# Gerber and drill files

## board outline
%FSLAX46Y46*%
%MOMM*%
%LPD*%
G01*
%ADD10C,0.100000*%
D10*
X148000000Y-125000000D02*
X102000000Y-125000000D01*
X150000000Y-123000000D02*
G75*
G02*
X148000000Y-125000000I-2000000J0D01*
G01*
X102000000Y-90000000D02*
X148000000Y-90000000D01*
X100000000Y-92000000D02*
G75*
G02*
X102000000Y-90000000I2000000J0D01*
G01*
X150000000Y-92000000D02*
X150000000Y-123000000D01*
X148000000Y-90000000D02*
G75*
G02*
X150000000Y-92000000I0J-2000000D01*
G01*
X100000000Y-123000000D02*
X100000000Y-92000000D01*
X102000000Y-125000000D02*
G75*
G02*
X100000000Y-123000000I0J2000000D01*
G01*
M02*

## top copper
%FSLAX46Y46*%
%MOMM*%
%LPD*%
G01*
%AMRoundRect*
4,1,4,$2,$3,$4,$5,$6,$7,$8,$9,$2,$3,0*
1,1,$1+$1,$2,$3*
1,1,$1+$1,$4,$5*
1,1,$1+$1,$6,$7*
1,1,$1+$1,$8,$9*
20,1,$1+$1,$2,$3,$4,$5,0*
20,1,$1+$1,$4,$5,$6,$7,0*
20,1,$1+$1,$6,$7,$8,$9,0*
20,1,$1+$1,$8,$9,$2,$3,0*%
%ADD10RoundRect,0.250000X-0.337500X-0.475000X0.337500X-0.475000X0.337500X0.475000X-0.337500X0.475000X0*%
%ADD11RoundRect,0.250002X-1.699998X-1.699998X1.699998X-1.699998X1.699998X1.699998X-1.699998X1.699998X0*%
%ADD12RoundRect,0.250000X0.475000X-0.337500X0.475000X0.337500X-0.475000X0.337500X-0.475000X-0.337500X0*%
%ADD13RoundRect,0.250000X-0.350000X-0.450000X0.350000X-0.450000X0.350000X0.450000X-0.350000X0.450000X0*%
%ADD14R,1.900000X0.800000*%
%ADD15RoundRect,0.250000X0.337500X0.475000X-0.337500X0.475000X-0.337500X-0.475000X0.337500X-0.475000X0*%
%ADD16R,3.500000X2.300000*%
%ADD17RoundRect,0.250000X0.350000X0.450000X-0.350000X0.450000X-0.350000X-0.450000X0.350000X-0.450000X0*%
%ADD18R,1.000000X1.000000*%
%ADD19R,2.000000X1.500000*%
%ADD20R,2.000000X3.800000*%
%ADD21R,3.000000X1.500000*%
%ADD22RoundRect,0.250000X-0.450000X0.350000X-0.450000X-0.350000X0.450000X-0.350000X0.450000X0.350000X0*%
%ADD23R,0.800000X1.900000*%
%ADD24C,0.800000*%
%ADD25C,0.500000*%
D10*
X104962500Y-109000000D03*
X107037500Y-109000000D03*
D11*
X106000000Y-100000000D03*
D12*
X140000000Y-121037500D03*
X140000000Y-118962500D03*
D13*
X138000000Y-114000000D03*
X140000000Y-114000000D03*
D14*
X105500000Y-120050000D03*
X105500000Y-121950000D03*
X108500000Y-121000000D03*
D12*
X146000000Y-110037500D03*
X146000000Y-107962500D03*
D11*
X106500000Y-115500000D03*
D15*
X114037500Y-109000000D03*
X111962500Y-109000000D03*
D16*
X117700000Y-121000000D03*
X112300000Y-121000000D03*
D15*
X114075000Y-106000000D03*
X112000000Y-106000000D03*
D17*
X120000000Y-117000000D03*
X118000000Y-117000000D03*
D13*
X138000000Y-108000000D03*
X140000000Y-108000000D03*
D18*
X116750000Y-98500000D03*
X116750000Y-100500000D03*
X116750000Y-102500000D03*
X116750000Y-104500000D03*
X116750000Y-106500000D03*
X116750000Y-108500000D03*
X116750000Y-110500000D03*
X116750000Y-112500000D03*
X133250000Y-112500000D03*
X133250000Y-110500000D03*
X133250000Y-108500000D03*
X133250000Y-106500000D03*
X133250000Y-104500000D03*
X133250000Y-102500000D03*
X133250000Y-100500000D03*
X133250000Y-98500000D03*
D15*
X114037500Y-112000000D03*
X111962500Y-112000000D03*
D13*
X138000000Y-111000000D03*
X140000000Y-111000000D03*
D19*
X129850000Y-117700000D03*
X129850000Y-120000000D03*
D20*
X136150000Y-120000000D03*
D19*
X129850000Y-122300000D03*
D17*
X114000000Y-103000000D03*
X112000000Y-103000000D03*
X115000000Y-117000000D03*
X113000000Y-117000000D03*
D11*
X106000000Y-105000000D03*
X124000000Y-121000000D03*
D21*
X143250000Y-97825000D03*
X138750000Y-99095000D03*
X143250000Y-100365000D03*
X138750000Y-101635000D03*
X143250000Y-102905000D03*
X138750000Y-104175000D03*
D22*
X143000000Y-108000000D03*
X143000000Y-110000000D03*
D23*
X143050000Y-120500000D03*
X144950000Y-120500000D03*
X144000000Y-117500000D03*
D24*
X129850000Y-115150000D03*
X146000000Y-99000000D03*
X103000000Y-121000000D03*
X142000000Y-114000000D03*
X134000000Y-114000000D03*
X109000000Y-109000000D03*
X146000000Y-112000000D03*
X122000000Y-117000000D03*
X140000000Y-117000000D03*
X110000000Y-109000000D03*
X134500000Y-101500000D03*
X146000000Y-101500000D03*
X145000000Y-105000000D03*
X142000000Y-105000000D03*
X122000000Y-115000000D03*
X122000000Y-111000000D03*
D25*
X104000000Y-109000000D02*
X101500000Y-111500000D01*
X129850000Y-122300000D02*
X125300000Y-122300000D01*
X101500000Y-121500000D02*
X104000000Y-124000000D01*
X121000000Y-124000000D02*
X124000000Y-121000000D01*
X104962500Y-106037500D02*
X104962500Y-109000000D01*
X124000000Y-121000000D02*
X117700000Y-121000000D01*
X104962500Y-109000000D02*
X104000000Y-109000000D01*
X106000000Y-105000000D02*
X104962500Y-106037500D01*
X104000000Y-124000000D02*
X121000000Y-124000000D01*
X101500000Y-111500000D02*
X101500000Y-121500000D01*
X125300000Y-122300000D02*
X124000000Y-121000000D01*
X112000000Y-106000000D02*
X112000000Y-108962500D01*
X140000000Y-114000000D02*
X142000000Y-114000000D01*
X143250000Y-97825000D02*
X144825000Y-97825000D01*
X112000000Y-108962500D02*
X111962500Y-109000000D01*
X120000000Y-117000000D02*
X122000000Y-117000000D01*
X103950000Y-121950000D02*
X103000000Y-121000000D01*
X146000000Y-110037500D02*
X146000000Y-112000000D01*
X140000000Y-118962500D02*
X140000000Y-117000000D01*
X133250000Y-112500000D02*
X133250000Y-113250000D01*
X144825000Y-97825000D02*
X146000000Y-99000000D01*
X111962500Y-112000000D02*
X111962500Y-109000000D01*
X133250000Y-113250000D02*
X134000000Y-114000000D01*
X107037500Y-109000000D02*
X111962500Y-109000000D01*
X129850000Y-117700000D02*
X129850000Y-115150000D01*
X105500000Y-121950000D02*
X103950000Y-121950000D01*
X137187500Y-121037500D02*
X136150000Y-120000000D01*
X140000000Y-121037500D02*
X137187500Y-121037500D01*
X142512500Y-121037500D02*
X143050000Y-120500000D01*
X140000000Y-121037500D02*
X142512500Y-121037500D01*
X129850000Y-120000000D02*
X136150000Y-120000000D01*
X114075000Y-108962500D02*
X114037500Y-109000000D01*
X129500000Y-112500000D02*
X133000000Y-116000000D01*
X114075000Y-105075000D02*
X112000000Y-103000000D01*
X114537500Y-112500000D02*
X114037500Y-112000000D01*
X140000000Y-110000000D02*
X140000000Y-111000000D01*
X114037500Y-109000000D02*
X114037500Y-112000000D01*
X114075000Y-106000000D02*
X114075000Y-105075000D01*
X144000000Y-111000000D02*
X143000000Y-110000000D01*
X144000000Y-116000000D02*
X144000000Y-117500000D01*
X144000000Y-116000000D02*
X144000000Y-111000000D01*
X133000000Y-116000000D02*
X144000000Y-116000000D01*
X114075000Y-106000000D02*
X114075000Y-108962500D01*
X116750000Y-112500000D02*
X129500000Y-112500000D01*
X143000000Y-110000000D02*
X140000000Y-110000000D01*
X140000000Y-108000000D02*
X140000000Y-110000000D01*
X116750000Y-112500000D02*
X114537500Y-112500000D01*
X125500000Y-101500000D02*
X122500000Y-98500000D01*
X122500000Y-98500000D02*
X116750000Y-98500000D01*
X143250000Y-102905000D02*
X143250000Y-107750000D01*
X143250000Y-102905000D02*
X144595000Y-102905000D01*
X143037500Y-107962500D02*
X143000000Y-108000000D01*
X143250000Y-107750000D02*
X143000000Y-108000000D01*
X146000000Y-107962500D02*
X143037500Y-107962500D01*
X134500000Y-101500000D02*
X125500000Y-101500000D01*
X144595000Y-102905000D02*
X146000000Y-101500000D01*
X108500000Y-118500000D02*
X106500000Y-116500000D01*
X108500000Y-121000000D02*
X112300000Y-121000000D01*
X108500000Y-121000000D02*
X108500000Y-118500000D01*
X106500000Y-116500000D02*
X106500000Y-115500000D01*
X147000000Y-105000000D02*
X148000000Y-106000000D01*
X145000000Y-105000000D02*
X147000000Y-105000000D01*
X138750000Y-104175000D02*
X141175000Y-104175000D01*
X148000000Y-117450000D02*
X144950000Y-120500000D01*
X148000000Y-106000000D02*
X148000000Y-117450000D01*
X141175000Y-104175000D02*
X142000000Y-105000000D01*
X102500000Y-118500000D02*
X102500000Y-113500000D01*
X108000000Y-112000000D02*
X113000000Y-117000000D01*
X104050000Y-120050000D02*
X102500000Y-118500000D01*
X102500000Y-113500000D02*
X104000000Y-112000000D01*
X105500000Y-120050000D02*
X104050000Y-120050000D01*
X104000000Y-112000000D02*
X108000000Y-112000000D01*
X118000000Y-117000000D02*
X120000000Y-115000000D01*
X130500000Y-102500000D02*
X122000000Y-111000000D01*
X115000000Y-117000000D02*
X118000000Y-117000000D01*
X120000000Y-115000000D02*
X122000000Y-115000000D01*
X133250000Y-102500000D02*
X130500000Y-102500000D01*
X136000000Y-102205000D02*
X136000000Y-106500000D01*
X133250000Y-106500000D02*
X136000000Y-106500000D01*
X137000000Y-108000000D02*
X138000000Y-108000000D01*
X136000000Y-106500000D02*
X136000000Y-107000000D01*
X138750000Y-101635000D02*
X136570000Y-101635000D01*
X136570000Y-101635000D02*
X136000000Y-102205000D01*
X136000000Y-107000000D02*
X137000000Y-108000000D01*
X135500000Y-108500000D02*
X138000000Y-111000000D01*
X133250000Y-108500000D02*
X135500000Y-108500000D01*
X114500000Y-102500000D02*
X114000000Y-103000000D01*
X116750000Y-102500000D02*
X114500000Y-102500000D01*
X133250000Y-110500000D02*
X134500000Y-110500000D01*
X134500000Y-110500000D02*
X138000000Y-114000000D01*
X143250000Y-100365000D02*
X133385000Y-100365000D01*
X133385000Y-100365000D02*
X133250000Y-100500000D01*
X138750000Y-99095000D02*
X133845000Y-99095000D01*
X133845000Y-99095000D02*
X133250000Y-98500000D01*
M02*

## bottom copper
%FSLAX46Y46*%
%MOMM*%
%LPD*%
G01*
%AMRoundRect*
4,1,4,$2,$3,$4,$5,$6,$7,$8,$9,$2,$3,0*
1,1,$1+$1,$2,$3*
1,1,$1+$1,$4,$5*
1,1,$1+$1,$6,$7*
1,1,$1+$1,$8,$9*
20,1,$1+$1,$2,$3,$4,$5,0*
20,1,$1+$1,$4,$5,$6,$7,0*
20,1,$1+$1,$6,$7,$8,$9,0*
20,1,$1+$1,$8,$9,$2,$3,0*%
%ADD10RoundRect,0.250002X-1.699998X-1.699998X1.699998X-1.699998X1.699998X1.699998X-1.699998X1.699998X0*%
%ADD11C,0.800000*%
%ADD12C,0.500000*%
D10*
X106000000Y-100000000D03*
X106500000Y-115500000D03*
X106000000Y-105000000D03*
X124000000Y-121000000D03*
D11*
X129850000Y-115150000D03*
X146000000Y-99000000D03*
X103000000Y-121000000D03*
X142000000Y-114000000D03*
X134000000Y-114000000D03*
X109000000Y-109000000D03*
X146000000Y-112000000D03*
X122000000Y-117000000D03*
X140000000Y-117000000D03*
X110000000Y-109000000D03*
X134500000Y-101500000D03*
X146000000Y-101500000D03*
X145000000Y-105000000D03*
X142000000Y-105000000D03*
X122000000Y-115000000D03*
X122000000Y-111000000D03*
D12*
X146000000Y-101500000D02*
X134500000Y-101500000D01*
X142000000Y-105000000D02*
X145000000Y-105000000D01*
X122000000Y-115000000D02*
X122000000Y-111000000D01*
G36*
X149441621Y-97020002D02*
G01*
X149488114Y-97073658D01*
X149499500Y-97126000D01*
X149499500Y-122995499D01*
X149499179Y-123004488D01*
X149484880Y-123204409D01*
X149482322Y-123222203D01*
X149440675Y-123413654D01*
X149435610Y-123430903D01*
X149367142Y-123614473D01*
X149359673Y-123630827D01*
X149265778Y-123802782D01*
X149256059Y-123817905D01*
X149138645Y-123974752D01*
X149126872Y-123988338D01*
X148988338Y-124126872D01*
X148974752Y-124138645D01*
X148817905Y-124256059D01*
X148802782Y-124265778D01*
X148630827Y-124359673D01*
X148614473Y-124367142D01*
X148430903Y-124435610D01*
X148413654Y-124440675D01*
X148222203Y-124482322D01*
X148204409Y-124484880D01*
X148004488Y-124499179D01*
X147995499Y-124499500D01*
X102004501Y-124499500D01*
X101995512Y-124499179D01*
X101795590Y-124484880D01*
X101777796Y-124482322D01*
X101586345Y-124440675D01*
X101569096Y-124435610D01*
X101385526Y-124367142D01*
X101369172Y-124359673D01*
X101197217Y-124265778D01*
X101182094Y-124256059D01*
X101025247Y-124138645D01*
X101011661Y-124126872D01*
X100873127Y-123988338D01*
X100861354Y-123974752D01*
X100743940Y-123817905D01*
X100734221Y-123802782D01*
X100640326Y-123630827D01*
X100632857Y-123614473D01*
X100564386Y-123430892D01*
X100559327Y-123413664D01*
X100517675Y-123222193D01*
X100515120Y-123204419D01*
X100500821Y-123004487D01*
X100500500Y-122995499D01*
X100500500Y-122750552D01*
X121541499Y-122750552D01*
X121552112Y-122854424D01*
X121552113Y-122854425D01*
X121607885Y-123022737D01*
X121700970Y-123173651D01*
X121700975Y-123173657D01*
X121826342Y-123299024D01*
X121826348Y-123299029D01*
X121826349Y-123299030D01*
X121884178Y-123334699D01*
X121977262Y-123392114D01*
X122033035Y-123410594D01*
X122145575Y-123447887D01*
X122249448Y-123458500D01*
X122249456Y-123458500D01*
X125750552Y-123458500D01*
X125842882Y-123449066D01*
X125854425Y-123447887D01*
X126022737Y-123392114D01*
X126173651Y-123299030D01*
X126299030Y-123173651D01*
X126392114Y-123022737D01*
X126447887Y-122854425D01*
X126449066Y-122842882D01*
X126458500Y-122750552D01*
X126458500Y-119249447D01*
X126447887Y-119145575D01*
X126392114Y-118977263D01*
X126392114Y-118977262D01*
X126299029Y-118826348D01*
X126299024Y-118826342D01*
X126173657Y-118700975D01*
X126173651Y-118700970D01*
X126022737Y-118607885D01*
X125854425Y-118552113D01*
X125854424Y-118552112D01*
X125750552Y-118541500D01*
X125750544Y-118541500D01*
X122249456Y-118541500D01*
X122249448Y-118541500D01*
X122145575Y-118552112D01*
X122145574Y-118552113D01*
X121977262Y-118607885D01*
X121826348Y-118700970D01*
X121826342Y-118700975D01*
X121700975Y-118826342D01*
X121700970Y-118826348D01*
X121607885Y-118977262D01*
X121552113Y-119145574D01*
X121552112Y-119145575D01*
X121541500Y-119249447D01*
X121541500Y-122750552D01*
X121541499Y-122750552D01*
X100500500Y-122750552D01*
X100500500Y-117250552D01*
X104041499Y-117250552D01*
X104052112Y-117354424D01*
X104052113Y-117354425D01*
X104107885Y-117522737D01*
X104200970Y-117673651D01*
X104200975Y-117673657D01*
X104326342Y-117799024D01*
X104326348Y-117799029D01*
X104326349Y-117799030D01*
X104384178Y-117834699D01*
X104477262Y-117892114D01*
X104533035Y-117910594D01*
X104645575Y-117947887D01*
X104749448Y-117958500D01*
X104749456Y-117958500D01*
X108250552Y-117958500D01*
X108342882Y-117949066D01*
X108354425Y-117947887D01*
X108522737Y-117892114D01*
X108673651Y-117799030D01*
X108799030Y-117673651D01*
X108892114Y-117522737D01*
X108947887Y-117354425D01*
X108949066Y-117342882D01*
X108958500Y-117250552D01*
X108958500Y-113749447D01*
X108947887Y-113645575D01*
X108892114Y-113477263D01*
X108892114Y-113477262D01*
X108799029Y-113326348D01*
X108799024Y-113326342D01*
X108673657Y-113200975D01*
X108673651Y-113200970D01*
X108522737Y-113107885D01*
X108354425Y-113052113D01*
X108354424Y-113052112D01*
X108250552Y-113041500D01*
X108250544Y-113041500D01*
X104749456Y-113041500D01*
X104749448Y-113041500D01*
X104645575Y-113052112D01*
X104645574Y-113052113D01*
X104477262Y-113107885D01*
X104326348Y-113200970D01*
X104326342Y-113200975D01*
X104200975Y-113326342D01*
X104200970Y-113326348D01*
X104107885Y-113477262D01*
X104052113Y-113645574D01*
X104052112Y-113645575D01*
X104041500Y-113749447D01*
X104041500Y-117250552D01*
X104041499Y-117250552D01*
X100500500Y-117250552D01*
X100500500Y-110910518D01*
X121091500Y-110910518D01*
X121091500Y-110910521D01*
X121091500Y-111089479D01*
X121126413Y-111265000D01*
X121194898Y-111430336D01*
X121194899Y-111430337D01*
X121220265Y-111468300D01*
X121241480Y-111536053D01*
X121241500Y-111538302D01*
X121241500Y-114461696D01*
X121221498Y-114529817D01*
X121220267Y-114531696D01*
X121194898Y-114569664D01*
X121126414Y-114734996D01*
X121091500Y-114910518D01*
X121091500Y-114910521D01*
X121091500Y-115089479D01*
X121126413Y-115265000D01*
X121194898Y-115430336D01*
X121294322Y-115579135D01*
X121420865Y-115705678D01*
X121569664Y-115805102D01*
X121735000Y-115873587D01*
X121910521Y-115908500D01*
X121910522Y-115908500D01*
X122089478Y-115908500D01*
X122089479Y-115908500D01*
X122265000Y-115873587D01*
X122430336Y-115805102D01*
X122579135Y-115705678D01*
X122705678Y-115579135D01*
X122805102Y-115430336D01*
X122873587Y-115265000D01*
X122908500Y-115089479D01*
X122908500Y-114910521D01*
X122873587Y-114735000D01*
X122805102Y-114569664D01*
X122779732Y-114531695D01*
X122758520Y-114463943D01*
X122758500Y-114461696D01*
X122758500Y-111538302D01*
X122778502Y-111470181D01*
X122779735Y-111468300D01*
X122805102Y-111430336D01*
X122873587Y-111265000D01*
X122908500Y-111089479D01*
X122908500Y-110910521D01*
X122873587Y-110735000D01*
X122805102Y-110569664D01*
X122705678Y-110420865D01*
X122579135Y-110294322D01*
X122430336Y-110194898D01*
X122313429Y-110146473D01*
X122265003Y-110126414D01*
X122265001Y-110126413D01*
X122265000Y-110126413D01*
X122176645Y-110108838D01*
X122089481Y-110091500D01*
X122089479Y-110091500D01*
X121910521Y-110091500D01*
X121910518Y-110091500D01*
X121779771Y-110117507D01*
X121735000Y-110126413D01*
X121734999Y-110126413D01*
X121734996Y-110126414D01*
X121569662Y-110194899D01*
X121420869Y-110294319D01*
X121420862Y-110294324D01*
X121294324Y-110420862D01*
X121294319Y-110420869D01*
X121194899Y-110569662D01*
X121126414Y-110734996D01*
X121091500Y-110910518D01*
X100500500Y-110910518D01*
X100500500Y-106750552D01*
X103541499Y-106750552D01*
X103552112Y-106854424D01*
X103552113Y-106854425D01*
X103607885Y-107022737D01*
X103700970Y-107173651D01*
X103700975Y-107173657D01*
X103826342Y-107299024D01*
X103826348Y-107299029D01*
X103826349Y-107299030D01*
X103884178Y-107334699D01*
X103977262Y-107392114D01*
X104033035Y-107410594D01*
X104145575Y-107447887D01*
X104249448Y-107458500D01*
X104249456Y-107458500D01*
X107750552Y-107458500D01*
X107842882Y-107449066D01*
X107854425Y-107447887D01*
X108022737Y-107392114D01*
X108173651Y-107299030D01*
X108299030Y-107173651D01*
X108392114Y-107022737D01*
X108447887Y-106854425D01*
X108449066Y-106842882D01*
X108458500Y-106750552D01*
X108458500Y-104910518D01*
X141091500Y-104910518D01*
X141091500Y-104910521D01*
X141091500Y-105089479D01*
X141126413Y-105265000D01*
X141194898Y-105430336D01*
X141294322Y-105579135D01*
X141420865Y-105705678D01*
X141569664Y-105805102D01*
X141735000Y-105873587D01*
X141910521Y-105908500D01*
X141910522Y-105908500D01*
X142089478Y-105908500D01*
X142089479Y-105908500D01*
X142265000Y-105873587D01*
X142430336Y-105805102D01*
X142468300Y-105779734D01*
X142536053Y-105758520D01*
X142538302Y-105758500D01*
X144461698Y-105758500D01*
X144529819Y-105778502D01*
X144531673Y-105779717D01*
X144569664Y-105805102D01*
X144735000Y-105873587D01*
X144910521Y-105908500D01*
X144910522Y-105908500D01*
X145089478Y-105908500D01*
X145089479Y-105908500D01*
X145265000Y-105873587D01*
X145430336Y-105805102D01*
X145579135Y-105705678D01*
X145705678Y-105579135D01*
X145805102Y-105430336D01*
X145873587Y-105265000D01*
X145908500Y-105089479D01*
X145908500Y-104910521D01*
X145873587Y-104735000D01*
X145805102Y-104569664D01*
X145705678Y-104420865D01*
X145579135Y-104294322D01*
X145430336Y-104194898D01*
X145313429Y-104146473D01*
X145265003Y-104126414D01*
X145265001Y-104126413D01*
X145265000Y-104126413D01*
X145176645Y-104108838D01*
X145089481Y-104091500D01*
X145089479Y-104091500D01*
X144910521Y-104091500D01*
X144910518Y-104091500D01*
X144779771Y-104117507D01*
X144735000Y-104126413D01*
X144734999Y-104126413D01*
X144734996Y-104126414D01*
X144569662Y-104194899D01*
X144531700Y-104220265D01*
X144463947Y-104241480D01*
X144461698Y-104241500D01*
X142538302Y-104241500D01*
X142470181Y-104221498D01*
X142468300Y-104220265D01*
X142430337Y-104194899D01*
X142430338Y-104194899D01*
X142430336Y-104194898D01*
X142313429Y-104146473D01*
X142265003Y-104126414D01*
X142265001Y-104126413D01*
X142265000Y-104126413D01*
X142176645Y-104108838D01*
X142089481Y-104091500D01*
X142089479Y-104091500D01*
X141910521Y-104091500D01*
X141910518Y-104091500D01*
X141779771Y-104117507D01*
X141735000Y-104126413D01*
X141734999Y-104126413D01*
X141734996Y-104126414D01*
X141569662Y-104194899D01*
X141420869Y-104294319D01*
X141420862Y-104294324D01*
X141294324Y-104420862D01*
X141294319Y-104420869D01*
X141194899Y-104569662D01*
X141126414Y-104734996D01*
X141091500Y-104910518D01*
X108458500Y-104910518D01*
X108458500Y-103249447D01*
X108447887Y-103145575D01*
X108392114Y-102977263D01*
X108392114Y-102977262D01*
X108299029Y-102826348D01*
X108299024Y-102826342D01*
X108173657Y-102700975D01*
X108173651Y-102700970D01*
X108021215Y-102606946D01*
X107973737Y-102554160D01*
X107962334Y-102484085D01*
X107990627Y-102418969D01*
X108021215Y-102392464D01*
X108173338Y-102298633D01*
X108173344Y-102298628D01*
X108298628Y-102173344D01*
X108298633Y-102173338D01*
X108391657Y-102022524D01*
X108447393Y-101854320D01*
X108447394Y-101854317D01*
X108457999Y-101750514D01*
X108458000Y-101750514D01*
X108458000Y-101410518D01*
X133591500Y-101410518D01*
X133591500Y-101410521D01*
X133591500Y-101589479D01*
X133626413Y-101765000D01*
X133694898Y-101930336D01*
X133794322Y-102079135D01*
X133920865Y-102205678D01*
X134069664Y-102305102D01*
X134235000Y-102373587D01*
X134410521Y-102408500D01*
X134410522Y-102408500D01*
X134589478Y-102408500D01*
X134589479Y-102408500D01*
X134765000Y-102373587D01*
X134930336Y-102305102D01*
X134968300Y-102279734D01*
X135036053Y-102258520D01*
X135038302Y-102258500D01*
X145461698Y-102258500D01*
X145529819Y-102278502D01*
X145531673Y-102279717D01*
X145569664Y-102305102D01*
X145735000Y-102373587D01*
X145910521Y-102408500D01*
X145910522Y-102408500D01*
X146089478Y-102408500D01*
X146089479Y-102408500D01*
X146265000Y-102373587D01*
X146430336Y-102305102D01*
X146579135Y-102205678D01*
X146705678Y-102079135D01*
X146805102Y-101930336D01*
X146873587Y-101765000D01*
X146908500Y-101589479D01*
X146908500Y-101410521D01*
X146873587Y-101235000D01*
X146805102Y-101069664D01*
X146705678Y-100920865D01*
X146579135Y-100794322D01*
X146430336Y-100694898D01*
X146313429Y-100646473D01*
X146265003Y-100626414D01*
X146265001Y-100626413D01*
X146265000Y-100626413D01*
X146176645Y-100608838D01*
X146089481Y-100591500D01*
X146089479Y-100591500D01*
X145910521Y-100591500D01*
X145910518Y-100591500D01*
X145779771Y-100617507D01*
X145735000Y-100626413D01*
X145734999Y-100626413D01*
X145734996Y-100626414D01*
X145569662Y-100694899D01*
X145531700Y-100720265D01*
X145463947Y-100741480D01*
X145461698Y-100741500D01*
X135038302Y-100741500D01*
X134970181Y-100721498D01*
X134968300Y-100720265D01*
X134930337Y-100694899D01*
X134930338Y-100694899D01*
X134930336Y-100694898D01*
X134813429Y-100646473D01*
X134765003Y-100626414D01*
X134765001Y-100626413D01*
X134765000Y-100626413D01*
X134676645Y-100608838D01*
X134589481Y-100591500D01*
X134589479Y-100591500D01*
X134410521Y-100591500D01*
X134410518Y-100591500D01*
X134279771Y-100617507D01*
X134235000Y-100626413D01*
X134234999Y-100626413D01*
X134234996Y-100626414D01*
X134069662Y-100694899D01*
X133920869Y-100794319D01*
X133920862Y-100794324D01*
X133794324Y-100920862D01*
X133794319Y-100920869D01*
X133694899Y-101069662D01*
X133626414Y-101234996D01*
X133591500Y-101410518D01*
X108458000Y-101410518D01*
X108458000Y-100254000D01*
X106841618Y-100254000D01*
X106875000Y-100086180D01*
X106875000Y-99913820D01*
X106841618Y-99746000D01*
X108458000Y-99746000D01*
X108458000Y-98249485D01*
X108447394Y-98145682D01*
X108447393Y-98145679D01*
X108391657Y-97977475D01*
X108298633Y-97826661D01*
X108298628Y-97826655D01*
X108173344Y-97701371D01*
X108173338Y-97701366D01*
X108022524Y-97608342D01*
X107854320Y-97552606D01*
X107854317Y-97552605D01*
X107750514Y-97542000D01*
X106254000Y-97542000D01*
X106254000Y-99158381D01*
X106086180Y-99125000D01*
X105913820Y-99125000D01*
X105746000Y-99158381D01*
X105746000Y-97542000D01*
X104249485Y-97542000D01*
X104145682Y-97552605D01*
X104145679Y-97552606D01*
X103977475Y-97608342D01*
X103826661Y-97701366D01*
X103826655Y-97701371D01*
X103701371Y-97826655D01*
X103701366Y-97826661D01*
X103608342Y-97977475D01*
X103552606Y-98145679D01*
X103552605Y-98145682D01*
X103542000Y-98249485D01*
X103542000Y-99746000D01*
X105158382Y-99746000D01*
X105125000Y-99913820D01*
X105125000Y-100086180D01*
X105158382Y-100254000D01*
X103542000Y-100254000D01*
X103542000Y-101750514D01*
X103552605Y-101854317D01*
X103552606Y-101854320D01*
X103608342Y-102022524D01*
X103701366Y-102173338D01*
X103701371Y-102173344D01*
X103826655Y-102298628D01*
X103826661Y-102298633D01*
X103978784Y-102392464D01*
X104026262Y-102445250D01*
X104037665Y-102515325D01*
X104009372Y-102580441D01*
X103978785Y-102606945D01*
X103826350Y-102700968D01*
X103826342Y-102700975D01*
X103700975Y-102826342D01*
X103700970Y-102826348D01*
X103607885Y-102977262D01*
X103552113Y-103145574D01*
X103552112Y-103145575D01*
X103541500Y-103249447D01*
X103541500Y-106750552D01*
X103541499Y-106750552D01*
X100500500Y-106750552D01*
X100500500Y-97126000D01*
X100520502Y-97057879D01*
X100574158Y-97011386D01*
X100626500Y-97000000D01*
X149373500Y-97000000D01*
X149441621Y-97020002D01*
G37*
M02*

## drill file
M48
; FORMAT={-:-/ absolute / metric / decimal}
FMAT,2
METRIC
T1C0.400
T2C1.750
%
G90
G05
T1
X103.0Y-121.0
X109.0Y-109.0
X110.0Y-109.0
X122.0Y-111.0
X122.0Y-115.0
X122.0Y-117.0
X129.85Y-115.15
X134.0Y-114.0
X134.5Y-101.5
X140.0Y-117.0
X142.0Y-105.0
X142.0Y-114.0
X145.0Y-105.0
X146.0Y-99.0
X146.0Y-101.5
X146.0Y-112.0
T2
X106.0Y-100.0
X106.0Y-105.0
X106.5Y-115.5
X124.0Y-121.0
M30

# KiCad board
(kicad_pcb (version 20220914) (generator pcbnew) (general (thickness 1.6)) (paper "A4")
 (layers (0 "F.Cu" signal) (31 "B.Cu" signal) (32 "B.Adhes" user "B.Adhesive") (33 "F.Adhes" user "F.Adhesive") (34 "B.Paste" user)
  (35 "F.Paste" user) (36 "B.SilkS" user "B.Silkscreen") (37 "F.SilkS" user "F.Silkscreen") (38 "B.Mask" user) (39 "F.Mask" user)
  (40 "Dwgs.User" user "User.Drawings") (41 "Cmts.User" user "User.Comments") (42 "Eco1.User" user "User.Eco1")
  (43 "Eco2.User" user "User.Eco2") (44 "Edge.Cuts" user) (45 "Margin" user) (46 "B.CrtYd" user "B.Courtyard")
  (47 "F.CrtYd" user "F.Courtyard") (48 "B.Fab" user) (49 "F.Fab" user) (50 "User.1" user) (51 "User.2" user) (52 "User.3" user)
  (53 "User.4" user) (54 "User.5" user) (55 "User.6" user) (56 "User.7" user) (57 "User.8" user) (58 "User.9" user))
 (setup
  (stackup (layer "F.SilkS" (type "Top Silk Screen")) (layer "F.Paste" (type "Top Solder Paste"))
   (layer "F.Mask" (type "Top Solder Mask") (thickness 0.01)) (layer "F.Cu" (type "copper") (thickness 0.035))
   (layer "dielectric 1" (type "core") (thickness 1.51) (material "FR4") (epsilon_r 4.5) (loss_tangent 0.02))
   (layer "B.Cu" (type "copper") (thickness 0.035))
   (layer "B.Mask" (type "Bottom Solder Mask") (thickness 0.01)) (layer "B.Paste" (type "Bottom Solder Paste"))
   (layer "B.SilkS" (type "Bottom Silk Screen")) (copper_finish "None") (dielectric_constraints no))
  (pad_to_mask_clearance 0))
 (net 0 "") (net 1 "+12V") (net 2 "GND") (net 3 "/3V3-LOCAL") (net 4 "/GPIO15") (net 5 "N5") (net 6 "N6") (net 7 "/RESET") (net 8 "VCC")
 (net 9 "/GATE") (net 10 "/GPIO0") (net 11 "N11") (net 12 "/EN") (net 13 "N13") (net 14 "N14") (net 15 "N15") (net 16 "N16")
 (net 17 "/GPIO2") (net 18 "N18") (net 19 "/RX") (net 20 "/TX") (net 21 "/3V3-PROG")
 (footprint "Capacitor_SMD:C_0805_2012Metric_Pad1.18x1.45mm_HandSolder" (layer "F.Cu") (at 106 109)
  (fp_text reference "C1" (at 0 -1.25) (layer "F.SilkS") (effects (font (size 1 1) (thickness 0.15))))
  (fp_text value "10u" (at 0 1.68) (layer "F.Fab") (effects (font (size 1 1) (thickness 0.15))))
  (pad "1" smd roundrect (at -1.0375 0) (size 1.175 1.45) (layers "F.Cu" "F.Paste" "F.Mask") (roundrect_rratio 0.212766) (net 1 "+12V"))
  (pad "2" smd roundrect (at 1.0375 0) (size 1.175 1.45) (layers "F.Cu" "F.Paste" "F.Mask") (roundrect_rratio 0.212766) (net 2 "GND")))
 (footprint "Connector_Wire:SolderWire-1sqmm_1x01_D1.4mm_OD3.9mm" (layer "F.Cu") (at 106 100)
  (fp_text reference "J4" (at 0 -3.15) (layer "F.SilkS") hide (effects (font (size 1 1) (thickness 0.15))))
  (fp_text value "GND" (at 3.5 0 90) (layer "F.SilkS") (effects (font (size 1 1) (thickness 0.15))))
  (pad "1" thru_hole roundrect (at 0 0) (size 3.9 3.9) (drill 1.75) (layers *.Cu *.Mask) (roundrect_rratio 0.064103) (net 2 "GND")))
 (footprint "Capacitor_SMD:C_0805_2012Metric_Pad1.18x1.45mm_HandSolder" (layer "F.Cu") (at 140 120 90)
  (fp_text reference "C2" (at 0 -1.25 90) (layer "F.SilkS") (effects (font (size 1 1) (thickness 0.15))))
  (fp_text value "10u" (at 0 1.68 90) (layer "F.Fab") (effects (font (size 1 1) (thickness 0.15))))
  (pad "1" smd roundrect (at -1.0375 0 90) (size 1.175 1.45) (layers "F.Cu" "F.Paste" "F.Mask") (roundrect_rratio 0.212766)
   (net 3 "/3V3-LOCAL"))
  (pad "2" smd roundrect (at 1.0375 0 90) (size 1.175 1.45) (layers "F.Cu" "F.Paste" "F.Mask") (roundrect_rratio 0.212766) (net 2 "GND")))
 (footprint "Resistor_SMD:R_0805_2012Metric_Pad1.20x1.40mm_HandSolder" (layer "F.Cu") (at 139 114)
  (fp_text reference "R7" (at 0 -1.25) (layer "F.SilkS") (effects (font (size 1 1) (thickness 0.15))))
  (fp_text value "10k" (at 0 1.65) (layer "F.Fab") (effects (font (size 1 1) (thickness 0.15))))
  (pad "1" smd roundrect (at -1 0) (size 1.2 1.4) (layers "F.Cu" "F.Paste" "F.Mask") (roundrect_rratio 0.208333) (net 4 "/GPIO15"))
  (pad "2" smd roundrect (at 1 0) (size 1.2 1.4) (layers "F.Cu" "F.Paste" "F.Mask") (roundrect_rratio 0.208333) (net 2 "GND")))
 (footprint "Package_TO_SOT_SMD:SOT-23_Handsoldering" (layer "F.Cu") (at 107 121)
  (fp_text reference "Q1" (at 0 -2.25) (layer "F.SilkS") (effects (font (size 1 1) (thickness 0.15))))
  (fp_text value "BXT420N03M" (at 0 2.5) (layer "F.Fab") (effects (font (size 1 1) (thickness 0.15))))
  (pad "1" smd rect (at -1.5 -0.95) (size 1.9 0.8) (layers "F.Cu" "F.Paste" "F.Mask") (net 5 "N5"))
  (pad "2" smd rect (at -1.5 0.95) (size 1.9 0.8) (layers "F.Cu" "F.Paste" "F.Mask") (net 2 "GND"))
  (pad "3" smd rect (at 1.5 0) (size 1.9 0.8) (layers "F.Cu" "F.Paste" "F.Mask") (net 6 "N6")))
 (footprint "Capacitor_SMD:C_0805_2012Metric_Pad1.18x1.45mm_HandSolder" (layer "F.Cu") (at 146 109 90)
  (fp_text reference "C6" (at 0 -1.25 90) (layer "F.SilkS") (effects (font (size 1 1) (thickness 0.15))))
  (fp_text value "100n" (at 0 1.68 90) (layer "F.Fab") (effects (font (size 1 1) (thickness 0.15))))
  (pad "1" smd roundrect (at -1.0375 0 90) (size 1.175 1.45) (layers "F.Cu" "F.Paste" "F.Mask") (roundrect_rratio 0.212766) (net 2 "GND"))
  (pad "2" smd roundrect (at 1.0375 0 90) (size 1.175 1.45) (layers "F.Cu" "F.Paste" "F.Mask") (roundrect_rratio 0.212766) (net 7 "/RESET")))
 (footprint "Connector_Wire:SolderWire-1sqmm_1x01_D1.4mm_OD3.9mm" (layer "F.Cu") (at 106.5 115.5)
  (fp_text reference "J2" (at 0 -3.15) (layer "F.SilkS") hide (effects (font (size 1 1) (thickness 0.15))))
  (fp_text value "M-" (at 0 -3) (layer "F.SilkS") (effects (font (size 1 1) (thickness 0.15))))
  (pad "1" thru_hole roundrect (at 0 0) (size 3.9 3.9) (drill 1.75) (layers *.Cu *.Mask) (roundrect_rratio 0.064103) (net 6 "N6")))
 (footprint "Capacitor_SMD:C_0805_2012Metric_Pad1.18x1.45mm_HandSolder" (layer "F.Cu") (at 113 109 180)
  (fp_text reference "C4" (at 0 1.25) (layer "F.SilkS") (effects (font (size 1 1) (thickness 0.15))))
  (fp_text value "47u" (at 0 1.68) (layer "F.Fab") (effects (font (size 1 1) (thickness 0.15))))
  (pad "1" smd roundrect (at -1.0375 0 180) (size 1.175 1.45) (layers "F.Cu" "F.Paste" "F.Mask") (roundrect_rratio 0.212766) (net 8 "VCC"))
  (pad "2" smd roundrect (at 1.0375 0 180) (size 1.175 1.45) (layers "F.Cu" "F.Paste" "F.Mask") (roundrect_rratio 0.212766) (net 2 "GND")))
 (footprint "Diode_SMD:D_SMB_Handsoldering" (layer "F.Cu") (at 115 121 180)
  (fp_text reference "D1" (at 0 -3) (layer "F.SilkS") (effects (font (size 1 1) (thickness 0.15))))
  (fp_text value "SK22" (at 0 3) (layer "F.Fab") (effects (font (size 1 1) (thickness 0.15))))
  (pad "1" smd rect (at -2.7 0 180) (size 3.5 2.3) (layers "F.Cu" "F.Paste" "F.Mask") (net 1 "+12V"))
  (pad "2" smd rect (at 2.7 0 180) (size 3.5 2.3) (layers "F.Cu" "F.Paste" "F.Mask") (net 6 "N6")))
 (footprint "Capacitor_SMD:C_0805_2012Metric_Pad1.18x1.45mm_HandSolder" (layer "F.Cu") (at 113.0375 106 180)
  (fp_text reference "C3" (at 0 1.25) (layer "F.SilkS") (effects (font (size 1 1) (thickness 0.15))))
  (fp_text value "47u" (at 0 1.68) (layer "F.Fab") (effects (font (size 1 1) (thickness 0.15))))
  (pad "1" smd roundrect (at -1.0375 0 180) (size 1.175 1.45) (layers "F.Cu" "F.Paste" "F.Mask") (roundrect_rratio 0.212766) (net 8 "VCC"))
  (pad "2" smd roundrect (at 1.0375 0 180) (size 1.175 1.45) (layers "F.Cu" "F.Paste" "F.Mask") (roundrect_rratio 0.212766) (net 2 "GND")))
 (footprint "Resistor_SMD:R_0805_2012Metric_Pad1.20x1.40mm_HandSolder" (layer "F.Cu") (at 119 117 180)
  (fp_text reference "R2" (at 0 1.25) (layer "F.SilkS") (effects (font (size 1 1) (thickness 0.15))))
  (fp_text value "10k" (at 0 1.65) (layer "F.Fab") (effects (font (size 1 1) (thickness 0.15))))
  (pad "1" smd roundrect (at -1 0 180) (size 1.2 1.4) (layers "F.Cu" "F.Paste" "F.Mask") (roundrect_rratio 0.208333) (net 2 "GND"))
  (pad "2" smd roundrect (at 1 0 180) (size 1.2 1.4) (layers "F.Cu" "F.Paste" "F.Mask") (roundrect_rratio 0.208333) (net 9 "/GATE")))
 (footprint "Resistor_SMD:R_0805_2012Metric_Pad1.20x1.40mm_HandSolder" (layer "F.Cu") (at 139 108)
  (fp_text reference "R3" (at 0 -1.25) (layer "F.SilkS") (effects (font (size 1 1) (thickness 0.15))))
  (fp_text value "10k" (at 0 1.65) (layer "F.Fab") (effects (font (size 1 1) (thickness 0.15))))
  (pad "1" smd roundrect (at -1 0) (size 1.2 1.4) (layers "F.Cu" "F.Paste" "F.Mask") (roundrect_rratio 0.208333) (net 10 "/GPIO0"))
  (pad "2" smd roundrect (at 1 0) (size 1.2 1.4) (layers "F.Cu" "F.Paste" "F.Mask") (roundrect_rratio 0.208333) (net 8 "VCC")))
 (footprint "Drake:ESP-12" (layer "F.Cu") (at 125 114)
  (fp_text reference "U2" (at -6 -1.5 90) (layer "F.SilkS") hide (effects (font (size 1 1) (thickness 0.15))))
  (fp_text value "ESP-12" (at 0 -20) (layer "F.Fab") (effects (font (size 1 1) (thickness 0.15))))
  (pad "1" smd rect (at -8.25 -15.5) (size 1 1) (layers "F.Cu" "F.Paste" "F.Mask") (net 7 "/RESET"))
  (pad "2" smd rect (at -8.25 -13.5) (size 1 1) (layers "F.Cu" "F.Paste" "F.Mask") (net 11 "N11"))
  (pad "3" smd rect (at -8.25 -11.5) (size 1 1) (layers "F.Cu" "F.Paste" "F.Mask") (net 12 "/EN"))
  (pad "4" smd rect (at -8.25 -9.5) (size 1 1) (layers "F.Cu" "F.Paste" "F.Mask") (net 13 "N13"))
  (pad "5" smd rect (at -8.25 -7.5) (size 1 1) (layers "F.Cu" "F.Paste" "F.Mask") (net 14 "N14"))
  (pad "6" smd rect (at -8.25 -5.5) (size 1 1) (layers "F.Cu" "F.Paste" "F.Mask") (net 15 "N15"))
  (pad "7" smd rect (at -8.25 -3.5) (size 1 1) (layers "F.Cu" "F.Paste" "F.Mask") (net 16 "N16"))
  (pad "8" smd rect (at -8.25 -1.5) (size 1 1) (layers "F.Cu" "F.Paste" "F.Mask") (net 8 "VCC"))
  (pad "9" smd rect (at 8.25 -1.5) (size 1 1) (layers "F.Cu" "F.Paste" "F.Mask") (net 2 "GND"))
  (pad "10" smd rect (at 8.25 -3.5) (size 1 1) (layers "F.Cu" "F.Paste" "F.Mask") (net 4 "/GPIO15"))
  (pad "11" smd rect (at 8.25 -5.5) (size 1 1) (layers "F.Cu" "F.Paste" "F.Mask") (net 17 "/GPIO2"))
  (pad "12" smd rect (at 8.25 -7.5) (size 1 1) (layers "F.Cu" "F.Paste" "F.Mask") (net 10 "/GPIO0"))
  (pad "13" smd rect (at 8.25 -9.5) (size 1 1) (layers "F.Cu" "F.Paste" "F.Mask") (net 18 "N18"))
  (pad "14" smd rect (at 8.25 -11.5) (size 1 1) (layers "F.Cu" "F.Paste" "F.Mask") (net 9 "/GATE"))
  (pad "15" smd rect (at 8.25 -13.5) (size 1 1) (layers "F.Cu" "F.Paste" "F.Mask") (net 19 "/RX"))
  (pad "16" smd rect (at 8.25 -15.5) (size 1 1) (layers "F.Cu" "F.Paste" "F.Mask") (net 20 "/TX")))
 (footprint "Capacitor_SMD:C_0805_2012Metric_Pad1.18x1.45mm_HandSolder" (layer "F.Cu") (at 113 112 180)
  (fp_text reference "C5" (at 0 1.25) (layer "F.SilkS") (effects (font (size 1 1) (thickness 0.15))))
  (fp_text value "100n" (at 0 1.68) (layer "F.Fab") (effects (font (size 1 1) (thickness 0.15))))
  (pad "1" smd roundrect (at -1.0375 0 180) (size 1.175 1.45) (layers "F.Cu" "F.Paste" "F.Mask") (roundrect_rratio 0.212766) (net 8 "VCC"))
  (pad "2" smd roundrect (at 1.0375 0 180) (size 1.175 1.45) (layers "F.Cu" "F.Paste" "F.Mask") (roundrect_rratio 0.212766) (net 2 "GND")))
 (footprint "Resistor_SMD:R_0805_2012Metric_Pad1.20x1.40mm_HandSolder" (layer "F.Cu") (at 139 111)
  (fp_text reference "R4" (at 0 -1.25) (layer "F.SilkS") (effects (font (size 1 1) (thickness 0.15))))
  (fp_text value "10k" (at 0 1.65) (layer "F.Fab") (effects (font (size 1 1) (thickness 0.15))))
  (pad "1" smd roundrect (at -1 0) (size 1.2 1.4) (layers "F.Cu" "F.Paste" "F.Mask") (roundrect_rratio 0.208333) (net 17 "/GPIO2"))
  (pad "2" smd roundrect (at 1 0) (size 1.2 1.4) (layers "F.Cu" "F.Paste" "F.Mask") (roundrect_rratio 0.208333) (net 8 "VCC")))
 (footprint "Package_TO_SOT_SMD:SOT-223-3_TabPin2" (layer "F.Cu") (at 133 120)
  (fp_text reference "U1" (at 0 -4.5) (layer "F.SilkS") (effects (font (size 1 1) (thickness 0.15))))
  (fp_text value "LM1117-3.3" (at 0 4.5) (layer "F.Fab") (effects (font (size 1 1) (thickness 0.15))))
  (pad "1" smd rect (at -3.15 -2.3) (size 2 1.5) (layers "F.Cu" "F.Paste" "F.Mask") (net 2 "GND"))
  (pad "2" smd rect (at -3.15 0) (size 2 1.5) (layers "F.Cu" "F.Paste" "F.Mask") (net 3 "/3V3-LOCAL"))
  (pad "2" smd rect (at 3.15 0) (size 2 3.8) (layers "F.Cu" "F.Paste" "F.Mask") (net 3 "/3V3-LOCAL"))
  (pad "3" smd rect (at -3.15 2.3) (size 2 1.5) (layers "F.Cu" "F.Paste" "F.Mask") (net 1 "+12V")))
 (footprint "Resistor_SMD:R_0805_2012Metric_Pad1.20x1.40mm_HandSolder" (layer "F.Cu") (at 113 103 180)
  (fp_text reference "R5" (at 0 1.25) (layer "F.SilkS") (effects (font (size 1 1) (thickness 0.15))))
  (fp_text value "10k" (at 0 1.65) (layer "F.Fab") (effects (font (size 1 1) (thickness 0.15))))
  (pad "1" smd roundrect (at -1 0 180) (size 1.2 1.4) (layers "F.Cu" "F.Paste" "F.Mask") (roundrect_rratio 0.208333) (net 12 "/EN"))
  (pad "2" smd roundrect (at 1 0 180) (size 1.2 1.4) (layers "F.Cu" "F.Paste" "F.Mask") (roundrect_rratio 0.208333) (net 8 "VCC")))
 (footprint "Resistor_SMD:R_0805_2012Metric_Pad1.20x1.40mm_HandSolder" (layer "F.Cu") (at 114 117 180)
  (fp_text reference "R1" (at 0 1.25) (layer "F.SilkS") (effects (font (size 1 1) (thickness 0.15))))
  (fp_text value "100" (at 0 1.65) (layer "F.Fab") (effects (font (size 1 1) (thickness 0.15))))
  (pad "1" smd roundrect (at -1 0 180) (size 1.2 1.4) (layers "F.Cu" "F.Paste" "F.Mask") (roundrect_rratio 0.208333) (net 9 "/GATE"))
  (pad "2" smd roundrect (at 1 0 180) (size 1.2 1.4) (layers "F.Cu" "F.Paste" "F.Mask") (roundrect_rratio 0.208333) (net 5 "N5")))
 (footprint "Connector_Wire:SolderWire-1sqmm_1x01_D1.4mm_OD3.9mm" (layer "F.Cu") (at 106 105)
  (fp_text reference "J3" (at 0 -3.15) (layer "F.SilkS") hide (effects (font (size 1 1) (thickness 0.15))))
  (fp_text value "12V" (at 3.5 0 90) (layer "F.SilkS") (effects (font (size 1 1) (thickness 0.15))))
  (pad "1" thru_hole roundrect (at 0 0) (size 3.9 3.9) (drill 1.75) (layers *.Cu *.Mask) (roundrect_rratio 0.064103) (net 1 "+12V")))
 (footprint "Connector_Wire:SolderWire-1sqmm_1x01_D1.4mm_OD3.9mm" (layer "F.Cu") (at 124 121)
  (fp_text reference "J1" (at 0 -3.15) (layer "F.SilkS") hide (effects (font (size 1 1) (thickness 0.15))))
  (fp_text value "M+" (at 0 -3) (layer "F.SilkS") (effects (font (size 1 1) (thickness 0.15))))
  (pad "1" thru_hole roundrect (at 0 0) (size 3.9 3.9) (drill 1.75) (layers *.Cu *.Mask) (roundrect_rratio 0.064103) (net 1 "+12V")))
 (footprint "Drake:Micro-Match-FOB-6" (layer "F.Cu") (at 141 101 -90)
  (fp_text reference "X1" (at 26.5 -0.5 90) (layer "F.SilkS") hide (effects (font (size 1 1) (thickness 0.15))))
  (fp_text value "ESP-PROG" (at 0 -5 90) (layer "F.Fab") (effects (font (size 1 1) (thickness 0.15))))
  (pad "1" smd rect (at -3.175 -2.25 270) (size 1.5 3) (layers "F.Cu" "F.Paste" "F.Mask") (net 2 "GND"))
  (pad "2" smd rect (at -1.905 2.25 270) (size 1.5 3) (layers "F.Cu" "F.Paste" "F.Mask") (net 20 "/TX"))
  (pad "3" smd rect (at -0.635 -2.25 270) (size 1.5 3) (layers "F.Cu" "F.Paste" "F.Mask") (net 19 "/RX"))
  (pad "4" smd rect (at 0.635 2.25 270) (size 1.5 3) (layers "F.Cu" "F.Paste" "F.Mask") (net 10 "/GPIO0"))
  (pad "5" smd rect (at 1.905 -2.25 270) (size 1.5 3) (layers "F.Cu" "F.Paste" "F.Mask") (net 7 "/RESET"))
  (pad "6" smd rect (at 3.175 2.25 270) (size 1.5 3) (layers "F.Cu" "F.Paste" "F.Mask") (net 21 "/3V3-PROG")))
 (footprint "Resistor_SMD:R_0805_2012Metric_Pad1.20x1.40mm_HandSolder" (layer "F.Cu") (at 143 109 -90)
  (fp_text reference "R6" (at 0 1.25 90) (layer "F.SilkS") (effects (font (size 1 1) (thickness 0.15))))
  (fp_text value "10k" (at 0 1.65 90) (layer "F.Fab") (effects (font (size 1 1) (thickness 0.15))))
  (pad "1" smd roundrect (at -1 0 270) (size 1.2 1.4) (layers "F.Cu" "F.Paste" "F.Mask") (roundrect_rratio 0.208333) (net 7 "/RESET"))
  (pad "2" smd roundrect (at 1 0 270) (size 1.2 1.4) (layers "F.Cu" "F.Paste" "F.Mask") (roundrect_rratio 0.208333) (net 8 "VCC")))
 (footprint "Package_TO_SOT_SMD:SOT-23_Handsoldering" (layer "F.Cu") (at 144 119 90)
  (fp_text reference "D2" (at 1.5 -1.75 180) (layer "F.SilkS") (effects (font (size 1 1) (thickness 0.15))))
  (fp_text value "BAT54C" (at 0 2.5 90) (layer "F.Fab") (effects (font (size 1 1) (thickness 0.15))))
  (pad "1" smd rect (at -1.5 -0.95 90) (size 1.9 0.8) (layers "F.Cu" "F.Paste" "F.Mask") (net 3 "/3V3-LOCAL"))
  (pad "2" smd rect (at -1.5 0.95 90) (size 1.9 0.8) (layers "F.Cu" "F.Paste" "F.Mask") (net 21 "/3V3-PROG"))
  (pad "3" smd rect (at 1.5 0 90) (size 1.9 0.8) (layers "F.Cu" "F.Paste" "F.Mask") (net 8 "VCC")))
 (gr_line (start 148 125) (end 102 125) (stroke (width 0.1) (type default)) (layer "Edge.Cuts"))
 (gr_arc (start 150 123) (mid 149.414214 124.414214) (end 148 125) (stroke (width 0.1) (type default)) (layer "Edge.Cuts"))
 (gr_line (start 102 90) (end 148 90) (stroke (width 0.1) (type default)) (layer "Edge.Cuts"))
 (gr_arc (start 100 92) (mid 100.585786 90.585786) (end 102 90) (stroke (width 0.1) (type default)) (layer "Edge.Cuts"))
 (gr_line (start 150 92) (end 150 123) (stroke (width 0.1) (type default)) (layer "Edge.Cuts"))
 (gr_arc (start 148 90) (mid 149.414214 90.585786) (end 150 92) (stroke (width 0.1) (type default)) (layer "Edge.Cuts"))
 (gr_line (start 100 123) (end 100 92) (stroke (width 0.1) (type default)) (layer "Edge.Cuts"))
 (gr_arc (start 102 125) (mid 100.585786 124.414214) (end 100 123) (stroke (width 0.1) (type default)) (layer "Edge.Cuts"))
 (segment (start 104 109) (end 101.5 111.5) (width 0.5) (layer "F.Cu") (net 1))
 (segment (start 129.85 122.3) (end 125.3 122.3) (width 0.5) (layer "F.Cu") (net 1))
 (segment (start 101.5 121.5) (end 104 124) (width 0.5) (layer "F.Cu") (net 1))
 (segment (start 121 124) (end 124 121) (width 0.5) (layer "F.Cu") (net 1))
 (segment (start 104.9625 106.0375) (end 104.9625 109) (width 0.5) (layer "F.Cu") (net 1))
 (segment (start 124 121) (end 117.7 121) (width 0.5) (layer "F.Cu") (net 1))
 (segment (start 104.9625 109) (end 104 109) (width 0.5) (layer "F.Cu") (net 1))
 (segment (start 106 105) (end 104.9625 106.0375) (width 0.5) (layer "F.Cu") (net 1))
 (segment (start 104 124) (end 121 124) (width 0.5) (layer "F.Cu") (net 1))
 (segment (start 101.5 111.5) (end 101.5 121.5) (width 0.5) (layer "F.Cu") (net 1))
 (segment (start 125.3 122.3) (end 124 121) (width 0.5) (layer "F.Cu") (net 1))
 (segment (start 112 106) (end 112 108.9625) (width 0.5) (layer "F.Cu") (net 2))
 (segment (start 140 114) (end 142 114) (width 0.5) (layer "F.Cu") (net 2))
 (segment (start 143.25 97.825) (end 144.825 97.825) (width 0.5) (layer "F.Cu") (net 2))
 (segment (start 112 108.9625) (end 111.9625 109) (width 0.5) (layer "F.Cu") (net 2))
 (segment (start 120 117) (end 122 117) (width 0.5) (layer "F.Cu") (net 2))
 (segment (start 103.95 121.95) (end 103 121) (width 0.5) (layer "F.Cu") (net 2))
 (segment (start 146 110.0375) (end 146 112) (width 0.5) (layer "F.Cu") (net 2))
 (segment (start 140 118.9625) (end 140 117) (width 0.5) (layer "F.Cu") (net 2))
 (segment (start 133.25 112.5) (end 133.25 113.25) (width 0.5) (layer "F.Cu") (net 2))
 (segment (start 144.825 97.825) (end 146 99) (width 0.5) (layer "F.Cu") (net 2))
 (segment (start 111.9625 112) (end 111.9625 109) (width 0.5) (layer "F.Cu") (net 2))
 (segment (start 133.25 113.25) (end 134 114) (width 0.5) (layer "F.Cu") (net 2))
 (segment (start 107.0375 109) (end 111.9625 109) (width 0.5) (layer "F.Cu") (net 2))
 (segment (start 129.85 117.7) (end 129.85 115.15) (width 0.5) (layer "F.Cu") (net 2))
 (segment (start 105.5 121.95) (end 103.95 121.95) (width 0.5) (layer "F.Cu") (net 2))
 (via (at 129.85 115.15) (size 0.8) (drill 0.4) (layers "F.Cu" "B.Cu") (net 2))
 (via (at 146 99) (size 0.8) (drill 0.4) (layers "F.Cu" "B.Cu") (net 2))
 (via (at 103 121) (size 0.8) (drill 0.4) (layers "F.Cu" "B.Cu") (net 2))
 (via (at 142 114) (size 0.8) (drill 0.4) (layers "F.Cu" "B.Cu") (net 2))
 (via (at 134 114) (size 0.8) (drill 0.4) (layers "F.Cu" "B.Cu") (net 2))
 (via (at 109 109) (size 0.8) (drill 0.4) (layers "F.Cu" "B.Cu") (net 2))
 (via (at 146 112) (size 0.8) (drill 0.4) (layers "F.Cu" "B.Cu") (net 2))
 (via (at 122 117) (size 0.8) (drill 0.4) (layers "F.Cu" "B.Cu") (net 2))
 (via (at 140 117) (size 0.8) (drill 0.4) (layers "F.Cu" "B.Cu") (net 2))
 (via (at 110 109) (size 0.8) (drill 0.4) (layers "F.Cu" "B.Cu") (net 2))
 (segment (start 137.1875 121.0375) (end 136.15 120) (width 0.5) (layer "F.Cu") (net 3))
 (segment (start 140 121.0375) (end 137.1875 121.0375) (width 0.5) (layer "F.Cu") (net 3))
 (segment (start 142.5125 121.0375) (end 143.05 120.5) (width 0.5) (layer "F.Cu") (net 3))
 (segment (start 140 121.0375) (end 142.5125 121.0375) (width 0.5) (layer "F.Cu") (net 3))
 (segment (start 129.85 120) (end 136.15 120) (width 0.5) (layer "F.Cu") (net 3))
 (segment (start 114.075 108.9625) (end 114.0375 109) (width 0.5) (layer "F.Cu") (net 8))
 (segment (start 129.5 112.5) (end 133 116) (width 0.5) (layer "F.Cu") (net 8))
 (segment (start 114.075 105.075) (end 112 103) (width 0.5) (layer "F.Cu") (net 8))
 (segment (start 114.5375 112.5) (end 114.0375 112) (width 0.5) (layer "F.Cu") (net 8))
 (segment (start 140 110) (end 140 111) (width 0.5) (layer "F.Cu") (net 8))
 (segment (start 114.0375 109) (end 114.0375 112) (width 0.5) (layer "F.Cu") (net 8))
 (segment (start 114.075 106) (end 114.075 105.075) (width 0.5) (layer "F.Cu") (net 8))
 (segment (start 144 111) (end 143 110) (width 0.5) (layer "F.Cu") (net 8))
 (segment (start 144 116) (end 144 117.5) (width 0.5) (layer "F.Cu") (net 8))
 (segment (start 144 116) (end 144 111) (width 0.5) (layer "F.Cu") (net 8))
 (segment (start 133 116) (end 144 116) (width 0.5) (layer "F.Cu") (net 8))
 (segment (start 114.075 106) (end 114.075 108.9625) (width 0.5) (layer "F.Cu") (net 8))
 (segment (start 116.75 112.5) (end 129.5 112.5) (width 0.5) (layer "F.Cu") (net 8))
 (segment (start 143 110) (end 140 110) (width 0.5) (layer "F.Cu") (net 8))
 (segment (start 140 108) (end 140 110) (width 0.5) (layer "F.Cu") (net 8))
 (segment (start 116.75 112.5) (end 114.5375 112.5) (width 0.5) (layer "F.Cu") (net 8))
 (segment (start 125.5 101.5) (end 122.5 98.5) (width 0.5) (layer "F.Cu") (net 7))
 (segment (start 122.5 98.5) (end 116.75 98.5) (width 0.5) (layer "F.Cu") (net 7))
 (segment (start 143.25 102.905) (end 143.25 107.75) (width 0.5) (layer "F.Cu") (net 7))
 (segment (start 143.25 102.905) (end 144.595 102.905) (width 0.5) (layer "F.Cu") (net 7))
 (segment (start 143.0375 107.9625) (end 143 108) (width 0.5) (layer "F.Cu") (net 7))
 (segment (start 143.25 107.75) (end 143 108) (width 0.5) (layer "F.Cu") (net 7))
 (segment (start 146 107.9625) (end 143.0375 107.9625) (width 0.5) (layer "F.Cu") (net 7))
 (segment (start 134.5 101.5) (end 125.5 101.5) (width 0.5) (layer "F.Cu") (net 7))
 (segment (start 144.595 102.905) (end 146 101.5) (width 0.5) (layer "F.Cu") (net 7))
 (via (at 134.5 101.5) (size 0.8) (drill 0.4) (layers "F.Cu" "B.Cu") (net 7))
 (via (at 146 101.5) (size 0.8) (drill 0.4) (layers "F.Cu" "B.Cu") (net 7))
 (segment (start 146 101.5) (end 134.5 101.5) (width 0.5) (layer "B.Cu") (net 7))
 (segment (start 108.5 118.5) (end 106.5 116.5) (width 0.5) (layer "F.Cu") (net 6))
 (segment (start 108.5 121) (end 112.3 121) (width 0.5) (layer "F.Cu") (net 6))
 (segment (start 108.5 121) (end 108.5 118.5) (width 0.5) (layer "F.Cu") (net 6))
 (segment (start 106.5 116.5) (end 106.5 115.5) (width 0.5) (layer "F.Cu") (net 6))
 (segment (start 147 105) (end 148 106) (width 0.5) (layer "F.Cu") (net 21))
 (segment (start 145 105) (end 147 105) (width 0.5) (layer "F.Cu") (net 21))
 (segment (start 138.75 104.175) (end 141.175 104.175) (width 0.5) (layer "F.Cu") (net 21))
 (segment (start 148 117.45) (end 144.95 120.5) (width 0.5) (layer "F.Cu") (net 21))
 (segment (start 148 106) (end 148 117.45) (width 0.5) (layer "F.Cu") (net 21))
 (segment (start 141.175 104.175) (end 142 105) (width 0.5) (layer "F.Cu") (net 21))
 (via (at 145 105) (size 0.8) (drill 0.4) (layers "F.Cu" "B.Cu") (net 21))
 (via (at 142 105) (size 0.8) (drill 0.4) (layers "F.Cu" "B.Cu") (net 21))
 (segment (start 142 105) (end 145 105) (width 0.5) (layer "B.Cu") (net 21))
 (segment (start 102.5 118.5) (end 102.5 113.5) (width 0.5) (layer "F.Cu") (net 5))
 (segment (start 108 112) (end 113 117) (width 0.5) (layer "F.Cu") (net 5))
 (segment (start 104.05 120.05) (end 102.5 118.5) (width 0.5) (layer "F.Cu") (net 5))
 (segment (start 102.5 113.5) (end 104 112) (width 0.5) (layer "F.Cu") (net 5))
 (segment (start 105.5 120.05) (end 104.05 120.05) (width 0.5) (layer "F.Cu") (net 5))
 (segment (start 104 112) (end 108 112) (width 0.5) (layer "F.Cu") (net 5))
 (segment (start 118 117) (end 120 115) (width 0.5) (layer "F.Cu") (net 9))
 (segment (start 130.5 102.5) (end 122 111) (width 0.5) (layer "F.Cu") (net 9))
 (segment (start 115 117) (end 118 117) (width 0.5) (layer "F.Cu") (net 9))
 (segment (start 120 115) (end 122 115) (width 0.5) (layer "F.Cu") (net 9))
 (segment (start 133.25 102.5) (end 130.5 102.5) (width 0.5) (layer "F.Cu") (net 9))
 (via (at 122 115) (size 0.8) (drill 0.4) (layers "F.Cu" "B.Cu") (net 9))
 (via (at 122 111) (size 0.8) (drill 0.4) (layers "F.Cu" "B.Cu") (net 9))
 (segment (start 122 115) (end 122 111) (width 0.5) (layer "B.Cu") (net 9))
 (segment (start 136 102.205) (end 136 106.5) (width 0.5) (layer "F.Cu") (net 10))
 (segment (start 133.25 106.5) (end 136 106.5) (width 0.5) (layer "F.Cu") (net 10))
 (segment (start 137 108) (end 138 108) (width 0.5) (layer "F.Cu") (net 10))
 (segment (start 136 106.5) (end 136 107) (width 0.5) (layer "F.Cu") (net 10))
 (segment (start 138.75 101.635) (end 136.57 101.635) (width 0.5) (layer "F.Cu") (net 10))
 (segment (start 136.57 101.635) (end 136 102.205) (width 0.5) (layer "F.Cu") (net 10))
 (segment (start 136 107) (end 137 108) (width 0.5) (layer "F.Cu") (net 10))
 (segment (start 135.5 108.5) (end 138 111) (width 0.5) (layer "F.Cu") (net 17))
 (segment (start 133.25 108.5) (end 135.5 108.5) (width 0.5) (layer "F.Cu") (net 17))
 (segment (start 114.5 102.5) (end 114 103) (width 0.5) (layer "F.Cu") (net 12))
 (segment (start 116.75 102.5) (end 114.5 102.5) (width 0.5) (layer "F.Cu") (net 12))
 (segment (start 133.25 110.5) (end 134.5 110.5) (width 0.5) (layer "F.Cu") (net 4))
 (segment (start 134.5 110.5) (end 138 114) (width 0.5) (layer "F.Cu") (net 4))
 (segment (start 143.25 100.365) (end 133.385 100.365) (width 0.5) (layer "F.Cu") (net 19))
 (segment (start 133.385 100.365) (end 133.25 100.5) (width 0.5) (layer "F.Cu") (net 19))
 (segment (start 138.75 99.095) (end 133.845 99.095) (width 0.5) (layer "F.Cu") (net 20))
 (segment (start 133.845 99.095) (end 133.25 98.5) (width 0.5) (layer "F.Cu") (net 20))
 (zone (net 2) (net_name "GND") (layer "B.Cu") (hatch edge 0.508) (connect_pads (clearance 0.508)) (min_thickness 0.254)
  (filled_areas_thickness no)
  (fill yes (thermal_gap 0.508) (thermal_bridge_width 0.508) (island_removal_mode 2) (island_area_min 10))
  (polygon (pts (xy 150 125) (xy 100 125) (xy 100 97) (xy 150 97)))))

